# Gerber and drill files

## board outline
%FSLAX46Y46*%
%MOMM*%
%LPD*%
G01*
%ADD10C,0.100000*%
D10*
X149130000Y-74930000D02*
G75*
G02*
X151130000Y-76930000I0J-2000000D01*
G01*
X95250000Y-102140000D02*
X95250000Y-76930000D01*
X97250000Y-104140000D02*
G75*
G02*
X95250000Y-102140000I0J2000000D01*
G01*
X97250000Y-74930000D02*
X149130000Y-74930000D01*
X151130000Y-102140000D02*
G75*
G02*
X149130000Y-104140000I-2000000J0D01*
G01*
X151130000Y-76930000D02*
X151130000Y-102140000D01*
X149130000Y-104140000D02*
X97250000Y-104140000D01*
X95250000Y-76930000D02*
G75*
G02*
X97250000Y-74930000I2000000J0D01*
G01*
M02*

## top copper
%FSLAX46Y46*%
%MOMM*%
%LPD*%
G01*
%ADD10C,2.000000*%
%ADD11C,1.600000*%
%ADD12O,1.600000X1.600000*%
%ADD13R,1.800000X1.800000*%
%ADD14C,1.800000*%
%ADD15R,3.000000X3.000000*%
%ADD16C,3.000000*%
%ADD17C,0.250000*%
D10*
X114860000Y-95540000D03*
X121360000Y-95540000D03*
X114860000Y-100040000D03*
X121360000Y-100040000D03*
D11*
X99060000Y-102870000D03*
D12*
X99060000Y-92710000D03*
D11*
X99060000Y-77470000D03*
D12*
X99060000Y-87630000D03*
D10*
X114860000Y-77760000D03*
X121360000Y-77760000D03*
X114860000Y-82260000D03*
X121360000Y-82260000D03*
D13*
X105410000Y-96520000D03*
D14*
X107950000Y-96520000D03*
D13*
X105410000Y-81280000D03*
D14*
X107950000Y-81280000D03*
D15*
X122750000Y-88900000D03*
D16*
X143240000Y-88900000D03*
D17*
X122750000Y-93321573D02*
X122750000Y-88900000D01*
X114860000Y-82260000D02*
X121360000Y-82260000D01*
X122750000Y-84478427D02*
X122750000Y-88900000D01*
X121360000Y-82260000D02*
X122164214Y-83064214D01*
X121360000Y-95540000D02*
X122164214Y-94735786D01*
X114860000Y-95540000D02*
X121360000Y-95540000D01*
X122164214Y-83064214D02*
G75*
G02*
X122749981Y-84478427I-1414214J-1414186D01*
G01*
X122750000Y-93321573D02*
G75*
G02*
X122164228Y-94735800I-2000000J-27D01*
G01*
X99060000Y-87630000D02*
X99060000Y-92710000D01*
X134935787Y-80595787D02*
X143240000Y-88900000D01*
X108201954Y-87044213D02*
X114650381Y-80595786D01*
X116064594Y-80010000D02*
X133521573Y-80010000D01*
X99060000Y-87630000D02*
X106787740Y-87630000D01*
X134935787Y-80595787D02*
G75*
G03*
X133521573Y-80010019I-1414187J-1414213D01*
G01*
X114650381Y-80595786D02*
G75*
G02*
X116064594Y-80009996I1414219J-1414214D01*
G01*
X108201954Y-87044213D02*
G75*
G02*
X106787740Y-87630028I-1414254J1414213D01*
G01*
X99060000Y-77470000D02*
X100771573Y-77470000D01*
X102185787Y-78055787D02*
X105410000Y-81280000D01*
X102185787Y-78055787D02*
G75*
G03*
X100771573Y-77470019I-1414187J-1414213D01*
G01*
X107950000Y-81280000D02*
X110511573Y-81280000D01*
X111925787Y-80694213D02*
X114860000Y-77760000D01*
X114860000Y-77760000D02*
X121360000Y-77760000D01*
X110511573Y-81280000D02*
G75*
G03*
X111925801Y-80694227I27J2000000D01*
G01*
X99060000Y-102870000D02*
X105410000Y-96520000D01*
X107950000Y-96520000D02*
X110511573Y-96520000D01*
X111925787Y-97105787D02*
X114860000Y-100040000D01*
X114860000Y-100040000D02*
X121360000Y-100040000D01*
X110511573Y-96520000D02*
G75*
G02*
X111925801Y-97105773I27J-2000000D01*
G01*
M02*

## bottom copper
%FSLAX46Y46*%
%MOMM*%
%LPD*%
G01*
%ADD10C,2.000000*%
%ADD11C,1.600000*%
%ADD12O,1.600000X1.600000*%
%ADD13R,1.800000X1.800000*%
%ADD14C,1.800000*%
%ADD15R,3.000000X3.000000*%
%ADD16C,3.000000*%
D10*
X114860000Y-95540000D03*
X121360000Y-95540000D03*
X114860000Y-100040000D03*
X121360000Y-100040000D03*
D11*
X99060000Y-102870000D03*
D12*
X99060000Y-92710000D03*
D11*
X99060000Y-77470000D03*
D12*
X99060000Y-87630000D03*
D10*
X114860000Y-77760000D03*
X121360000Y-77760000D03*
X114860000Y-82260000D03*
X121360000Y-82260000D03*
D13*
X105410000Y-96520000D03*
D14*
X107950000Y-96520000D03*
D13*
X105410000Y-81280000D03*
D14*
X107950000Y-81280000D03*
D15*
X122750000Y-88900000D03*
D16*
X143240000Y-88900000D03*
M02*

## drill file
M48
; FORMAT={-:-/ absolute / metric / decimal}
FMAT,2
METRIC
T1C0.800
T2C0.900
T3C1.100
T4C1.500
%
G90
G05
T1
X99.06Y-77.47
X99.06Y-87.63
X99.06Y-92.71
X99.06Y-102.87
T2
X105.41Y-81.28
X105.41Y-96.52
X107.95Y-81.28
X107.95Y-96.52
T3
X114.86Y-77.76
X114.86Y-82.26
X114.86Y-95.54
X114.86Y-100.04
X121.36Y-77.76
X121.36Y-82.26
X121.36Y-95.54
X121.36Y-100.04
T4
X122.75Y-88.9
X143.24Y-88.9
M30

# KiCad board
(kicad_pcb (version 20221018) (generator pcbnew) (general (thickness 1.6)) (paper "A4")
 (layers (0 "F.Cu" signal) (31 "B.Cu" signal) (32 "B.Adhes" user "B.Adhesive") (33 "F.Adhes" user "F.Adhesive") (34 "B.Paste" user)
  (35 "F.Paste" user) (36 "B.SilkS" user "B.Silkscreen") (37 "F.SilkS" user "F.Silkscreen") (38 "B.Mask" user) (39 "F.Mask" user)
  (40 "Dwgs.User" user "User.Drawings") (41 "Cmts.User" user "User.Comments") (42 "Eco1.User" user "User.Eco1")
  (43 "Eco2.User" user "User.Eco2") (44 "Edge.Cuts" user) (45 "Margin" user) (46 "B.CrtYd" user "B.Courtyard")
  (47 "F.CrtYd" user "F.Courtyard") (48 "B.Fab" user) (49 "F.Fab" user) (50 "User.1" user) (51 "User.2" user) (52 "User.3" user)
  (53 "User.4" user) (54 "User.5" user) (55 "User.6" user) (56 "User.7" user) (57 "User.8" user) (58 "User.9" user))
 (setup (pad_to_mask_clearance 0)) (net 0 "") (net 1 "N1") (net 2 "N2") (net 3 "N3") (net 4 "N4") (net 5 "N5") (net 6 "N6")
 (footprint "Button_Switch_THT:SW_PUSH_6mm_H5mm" (layer "F.Cu") (at 114.86 95.54)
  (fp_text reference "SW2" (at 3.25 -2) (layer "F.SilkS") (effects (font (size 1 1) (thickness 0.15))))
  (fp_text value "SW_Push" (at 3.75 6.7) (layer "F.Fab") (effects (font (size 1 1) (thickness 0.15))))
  (pad "1" thru_hole circle (at 0 0 90) (size 2 2) (drill 1.1) (layers "*.Cu" "*.Mask") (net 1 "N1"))
  (pad "1" thru_hole circle (at 6.5 0 90) (size 2 2) (drill 1.1) (layers "*.Cu" "*.Mask") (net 1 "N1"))
  (pad "2" thru_hole circle (at 0 4.5 90) (size 2 2) (drill 1.1) (layers "*.Cu" "*.Mask") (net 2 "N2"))
  (pad "2" thru_hole circle (at 6.5 4.5 90) (size 2 2) (drill 1.1) (layers "*.Cu" "*.Mask") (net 2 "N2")))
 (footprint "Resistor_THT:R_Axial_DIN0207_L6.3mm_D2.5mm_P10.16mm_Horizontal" (layer "F.Cu") (at 99.06 102.87 90)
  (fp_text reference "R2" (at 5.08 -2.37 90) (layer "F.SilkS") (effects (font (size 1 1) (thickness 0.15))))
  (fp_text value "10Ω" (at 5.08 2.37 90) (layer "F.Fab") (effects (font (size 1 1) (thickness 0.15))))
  (pad "1" thru_hole circle (at 0 0 90) (size 1.6 1.6) (drill 0.8) (layers "*.Cu" "*.Mask") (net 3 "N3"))
  (pad "2" thru_hole oval (at 10.16 0 90) (size 1.6 1.6) (drill 0.8) (layers "*.Cu" "*.Mask") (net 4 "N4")))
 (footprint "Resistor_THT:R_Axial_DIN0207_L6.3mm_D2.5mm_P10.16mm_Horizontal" (layer "F.Cu") (at 99.06 77.47 -90)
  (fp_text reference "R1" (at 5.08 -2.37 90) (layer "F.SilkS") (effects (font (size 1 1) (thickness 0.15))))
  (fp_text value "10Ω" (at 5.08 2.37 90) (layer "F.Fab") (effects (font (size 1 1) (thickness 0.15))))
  (pad "1" thru_hole circle (at 0 0 270) (size 1.6 1.6) (drill 0.8) (layers "*.Cu" "*.Mask") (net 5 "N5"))
  (pad "2" thru_hole oval (at 10.16 0 270) (size 1.6 1.6) (drill 0.8) (layers "*.Cu" "*.Mask") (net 4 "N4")))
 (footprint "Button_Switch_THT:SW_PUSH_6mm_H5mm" (layer "F.Cu") (at 114.86 77.76)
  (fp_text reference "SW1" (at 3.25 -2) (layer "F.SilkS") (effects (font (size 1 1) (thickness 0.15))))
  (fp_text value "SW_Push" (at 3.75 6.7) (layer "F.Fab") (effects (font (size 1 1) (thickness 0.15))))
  (pad "1" thru_hole circle (at 0 0 90) (size 2 2) (drill 1.1) (layers "*.Cu" "*.Mask") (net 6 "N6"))
  (pad "1" thru_hole circle (at 6.5 0 90) (size 2 2) (drill 1.1) (layers "*.Cu" "*.Mask") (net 6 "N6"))
  (pad "2" thru_hole circle (at 0 4.5 90) (size 2 2) (drill 1.1) (layers "*.Cu" "*.Mask") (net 1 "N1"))
  (pad "2" thru_hole circle (at 6.5 4.5 90) (size 2 2) (drill 1.1) (layers "*.Cu" "*.Mask") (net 1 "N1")))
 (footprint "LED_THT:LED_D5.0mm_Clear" (layer "F.Cu") (at 105.41 96.52)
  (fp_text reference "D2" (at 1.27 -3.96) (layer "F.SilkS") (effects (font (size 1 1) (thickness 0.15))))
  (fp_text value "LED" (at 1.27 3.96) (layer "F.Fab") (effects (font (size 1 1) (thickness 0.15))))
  (pad "1" thru_hole rect (at 0 0) (size 1.8 1.8) (drill 0.9) (layers "*.Cu" "*.Mask") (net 3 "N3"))
  (pad "2" thru_hole circle (at 2.54 0) (size 1.8 1.8) (drill 0.9) (layers "*.Cu" "*.Mask") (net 2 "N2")))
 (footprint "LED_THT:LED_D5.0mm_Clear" (layer "F.Cu") (at 105.41 81.28)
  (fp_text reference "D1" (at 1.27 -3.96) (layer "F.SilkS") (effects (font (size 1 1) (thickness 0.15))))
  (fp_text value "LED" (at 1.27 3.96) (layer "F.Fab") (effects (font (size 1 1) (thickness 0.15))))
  (pad "1" thru_hole rect (at 0 0) (size 1.8 1.8) (drill 0.9) (layers "*.Cu" "*.Mask") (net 5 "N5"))
  (pad "2" thru_hole circle (at 2.54 0) (size 1.8 1.8) (drill 0.9) (layers "*.Cu" "*.Mask") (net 6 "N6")))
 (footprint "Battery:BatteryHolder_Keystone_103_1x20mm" (layer "F.Cu") (at 122.75 88.9)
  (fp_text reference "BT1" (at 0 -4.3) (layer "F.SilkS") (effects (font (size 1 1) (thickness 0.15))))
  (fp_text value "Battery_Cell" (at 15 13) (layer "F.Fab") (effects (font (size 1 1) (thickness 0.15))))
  (pad "1" thru_hole rect (at 0 0) (size 3 3) (drill 1.5) (layers "*.Cu" "*.Mask") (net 1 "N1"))
  (pad "2" thru_hole circle (at 20.49 0) (size 3 3) (drill 1.5) (layers "*.Cu" "*.Mask") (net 4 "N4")))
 (gr_arc (start 149.13 74.93) (mid 150.544214 75.515786) (end 151.13 76.93) (stroke (width 0.1) (type default)) (layer "Edge.Cuts"))
 (gr_line (start 95.25 102.14) (end 95.25 76.93) (stroke (width 0.1) (type default)) (layer "Edge.Cuts"))
 (gr_arc (start 97.25 104.14) (mid 95.835786 103.554214) (end 95.25 102.14) (stroke (width 0.1) (type default)) (layer "Edge.Cuts"))
 (gr_line (start 97.25 74.93) (end 149.13 74.93) (stroke (width 0.1) (type default)) (layer "Edge.Cuts"))
 (gr_arc (start 151.13 102.14) (mid 150.544214 103.554214) (end 149.13 104.14) (stroke (width 0.1) (type default)) (layer "Edge.Cuts"))
 (gr_line (start 151.13 76.93) (end 151.13 102.14) (stroke (width 0.1) (type default)) (layer "Edge.Cuts"))
 (gr_line (start 149.13 104.14) (end 97.25 104.14) (stroke (width 0.1) (type default)) (layer "Edge.Cuts"))
 (gr_arc (start 95.25 76.93) (mid 95.835786 75.515786) (end 97.25 74.93) (stroke (width 0.1) (type default)) (layer "Edge.Cuts"))
 (segment (start 122.75 93.321573) (end 122.75 88.9) (width 0.25) (layer "F.Cu") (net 1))
 (segment (start 114.86 82.26) (end 121.36 82.26) (width 0.25) (layer "F.Cu") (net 1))
 (segment (start 122.75 84.478427) (end 122.75 88.9) (width 0.25) (layer "F.Cu") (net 1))
 (segment (start 121.36 82.26) (end 122.164214 83.064214) (width 0.25) (layer "F.Cu") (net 1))
 (segment (start 121.36 95.54) (end 122.164214 94.735786) (width 0.25) (layer "F.Cu") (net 1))
 (segment (start 114.86 95.54) (end 121.36 95.54) (width 0.25) (layer "F.Cu") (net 1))
 (arc (start 122.164214 83.064214) (mid 122.597759 83.71306) (end 122.75 84.478427) (width 0.25) (layer "F.Cu") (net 1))
 (arc (start 122.75 93.321573) (mid 122.597759 94.08694) (end 122.164214 94.735786) (width 0.25) (layer "F.Cu") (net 1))
 (segment (start 99.06 87.63) (end 99.06 92.71) (width 0.25) (layer "F.Cu") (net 4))
 (segment (start 134.935787 80.595787) (end 143.24 88.9) (width 0.25) (layer "F.Cu") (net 4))
 (segment (start 108.201954 87.044213) (end 114.650381 80.595786) (width 0.25) (layer "F.Cu") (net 4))
 (segment (start 116.064594 80.01) (end 133.521573 80.01) (width 0.25) (layer "F.Cu") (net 4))
 (segment (start 99.06 87.63) (end 106.78774 87.63) (width 0.25) (layer "F.Cu") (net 4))
 (arc (start 134.935787 80.595787) (mid 134.28694 80.162241) (end 133.521573 80.01) (width 0.25) (layer "F.Cu") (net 4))
 (arc (start 114.650381 80.595786) (mid 115.299227 80.162241) (end 116.064594 80.01) (width 0.25) (layer "F.Cu") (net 4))
 (arc (start 108.201954 87.044213) (mid 107.553107 87.477759) (end 106.78774 87.63) (width 0.25) (layer "F.Cu") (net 4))
 (segment (start 99.06 77.47) (end 100.771573 77.47) (width 0.25) (layer "F.Cu") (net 5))
 (segment (start 102.185787 78.055787) (end 105.41 81.28) (width 0.25) (layer "F.Cu") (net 5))
 (arc (start 102.185787 78.055787) (mid 101.53694 77.622241) (end 100.771573 77.47) (width 0.25) (layer "F.Cu") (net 5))
 (segment (start 107.95 81.28) (end 110.511573 81.28) (width 0.25) (layer "F.Cu") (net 6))
 (segment (start 111.925787 80.694213) (end 114.86 77.76) (width 0.25) (layer "F.Cu") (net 6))
 (segment (start 114.86 77.76) (end 121.36 77.76) (width 0.25) (layer "F.Cu") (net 6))
 (arc (start 110.511573 81.28) (mid 111.27694 81.127759) (end 111.925787 80.694213) (width 0.25) (layer "F.Cu") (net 6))
 (segment (start 99.06 102.87) (end 105.41 96.52) (width 0.25) (layer "F.Cu") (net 3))
 (segment (start 107.95 96.52) (end 110.511573 96.52) (width 0.25) (layer "F.Cu") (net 2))
 (segment (start 111.925787 97.105787) (end 114.86 100.04) (width 0.25) (layer "F.Cu") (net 2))
 (segment (start 114.86 100.04) (end 121.36 100.04) (width 0.25) (layer "F.Cu") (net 2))
 (arc (start 110.511573 96.52) (mid 111.27694 96.672241) (end 111.925787 97.105787) (width 0.25) (layer "F.Cu") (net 2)))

